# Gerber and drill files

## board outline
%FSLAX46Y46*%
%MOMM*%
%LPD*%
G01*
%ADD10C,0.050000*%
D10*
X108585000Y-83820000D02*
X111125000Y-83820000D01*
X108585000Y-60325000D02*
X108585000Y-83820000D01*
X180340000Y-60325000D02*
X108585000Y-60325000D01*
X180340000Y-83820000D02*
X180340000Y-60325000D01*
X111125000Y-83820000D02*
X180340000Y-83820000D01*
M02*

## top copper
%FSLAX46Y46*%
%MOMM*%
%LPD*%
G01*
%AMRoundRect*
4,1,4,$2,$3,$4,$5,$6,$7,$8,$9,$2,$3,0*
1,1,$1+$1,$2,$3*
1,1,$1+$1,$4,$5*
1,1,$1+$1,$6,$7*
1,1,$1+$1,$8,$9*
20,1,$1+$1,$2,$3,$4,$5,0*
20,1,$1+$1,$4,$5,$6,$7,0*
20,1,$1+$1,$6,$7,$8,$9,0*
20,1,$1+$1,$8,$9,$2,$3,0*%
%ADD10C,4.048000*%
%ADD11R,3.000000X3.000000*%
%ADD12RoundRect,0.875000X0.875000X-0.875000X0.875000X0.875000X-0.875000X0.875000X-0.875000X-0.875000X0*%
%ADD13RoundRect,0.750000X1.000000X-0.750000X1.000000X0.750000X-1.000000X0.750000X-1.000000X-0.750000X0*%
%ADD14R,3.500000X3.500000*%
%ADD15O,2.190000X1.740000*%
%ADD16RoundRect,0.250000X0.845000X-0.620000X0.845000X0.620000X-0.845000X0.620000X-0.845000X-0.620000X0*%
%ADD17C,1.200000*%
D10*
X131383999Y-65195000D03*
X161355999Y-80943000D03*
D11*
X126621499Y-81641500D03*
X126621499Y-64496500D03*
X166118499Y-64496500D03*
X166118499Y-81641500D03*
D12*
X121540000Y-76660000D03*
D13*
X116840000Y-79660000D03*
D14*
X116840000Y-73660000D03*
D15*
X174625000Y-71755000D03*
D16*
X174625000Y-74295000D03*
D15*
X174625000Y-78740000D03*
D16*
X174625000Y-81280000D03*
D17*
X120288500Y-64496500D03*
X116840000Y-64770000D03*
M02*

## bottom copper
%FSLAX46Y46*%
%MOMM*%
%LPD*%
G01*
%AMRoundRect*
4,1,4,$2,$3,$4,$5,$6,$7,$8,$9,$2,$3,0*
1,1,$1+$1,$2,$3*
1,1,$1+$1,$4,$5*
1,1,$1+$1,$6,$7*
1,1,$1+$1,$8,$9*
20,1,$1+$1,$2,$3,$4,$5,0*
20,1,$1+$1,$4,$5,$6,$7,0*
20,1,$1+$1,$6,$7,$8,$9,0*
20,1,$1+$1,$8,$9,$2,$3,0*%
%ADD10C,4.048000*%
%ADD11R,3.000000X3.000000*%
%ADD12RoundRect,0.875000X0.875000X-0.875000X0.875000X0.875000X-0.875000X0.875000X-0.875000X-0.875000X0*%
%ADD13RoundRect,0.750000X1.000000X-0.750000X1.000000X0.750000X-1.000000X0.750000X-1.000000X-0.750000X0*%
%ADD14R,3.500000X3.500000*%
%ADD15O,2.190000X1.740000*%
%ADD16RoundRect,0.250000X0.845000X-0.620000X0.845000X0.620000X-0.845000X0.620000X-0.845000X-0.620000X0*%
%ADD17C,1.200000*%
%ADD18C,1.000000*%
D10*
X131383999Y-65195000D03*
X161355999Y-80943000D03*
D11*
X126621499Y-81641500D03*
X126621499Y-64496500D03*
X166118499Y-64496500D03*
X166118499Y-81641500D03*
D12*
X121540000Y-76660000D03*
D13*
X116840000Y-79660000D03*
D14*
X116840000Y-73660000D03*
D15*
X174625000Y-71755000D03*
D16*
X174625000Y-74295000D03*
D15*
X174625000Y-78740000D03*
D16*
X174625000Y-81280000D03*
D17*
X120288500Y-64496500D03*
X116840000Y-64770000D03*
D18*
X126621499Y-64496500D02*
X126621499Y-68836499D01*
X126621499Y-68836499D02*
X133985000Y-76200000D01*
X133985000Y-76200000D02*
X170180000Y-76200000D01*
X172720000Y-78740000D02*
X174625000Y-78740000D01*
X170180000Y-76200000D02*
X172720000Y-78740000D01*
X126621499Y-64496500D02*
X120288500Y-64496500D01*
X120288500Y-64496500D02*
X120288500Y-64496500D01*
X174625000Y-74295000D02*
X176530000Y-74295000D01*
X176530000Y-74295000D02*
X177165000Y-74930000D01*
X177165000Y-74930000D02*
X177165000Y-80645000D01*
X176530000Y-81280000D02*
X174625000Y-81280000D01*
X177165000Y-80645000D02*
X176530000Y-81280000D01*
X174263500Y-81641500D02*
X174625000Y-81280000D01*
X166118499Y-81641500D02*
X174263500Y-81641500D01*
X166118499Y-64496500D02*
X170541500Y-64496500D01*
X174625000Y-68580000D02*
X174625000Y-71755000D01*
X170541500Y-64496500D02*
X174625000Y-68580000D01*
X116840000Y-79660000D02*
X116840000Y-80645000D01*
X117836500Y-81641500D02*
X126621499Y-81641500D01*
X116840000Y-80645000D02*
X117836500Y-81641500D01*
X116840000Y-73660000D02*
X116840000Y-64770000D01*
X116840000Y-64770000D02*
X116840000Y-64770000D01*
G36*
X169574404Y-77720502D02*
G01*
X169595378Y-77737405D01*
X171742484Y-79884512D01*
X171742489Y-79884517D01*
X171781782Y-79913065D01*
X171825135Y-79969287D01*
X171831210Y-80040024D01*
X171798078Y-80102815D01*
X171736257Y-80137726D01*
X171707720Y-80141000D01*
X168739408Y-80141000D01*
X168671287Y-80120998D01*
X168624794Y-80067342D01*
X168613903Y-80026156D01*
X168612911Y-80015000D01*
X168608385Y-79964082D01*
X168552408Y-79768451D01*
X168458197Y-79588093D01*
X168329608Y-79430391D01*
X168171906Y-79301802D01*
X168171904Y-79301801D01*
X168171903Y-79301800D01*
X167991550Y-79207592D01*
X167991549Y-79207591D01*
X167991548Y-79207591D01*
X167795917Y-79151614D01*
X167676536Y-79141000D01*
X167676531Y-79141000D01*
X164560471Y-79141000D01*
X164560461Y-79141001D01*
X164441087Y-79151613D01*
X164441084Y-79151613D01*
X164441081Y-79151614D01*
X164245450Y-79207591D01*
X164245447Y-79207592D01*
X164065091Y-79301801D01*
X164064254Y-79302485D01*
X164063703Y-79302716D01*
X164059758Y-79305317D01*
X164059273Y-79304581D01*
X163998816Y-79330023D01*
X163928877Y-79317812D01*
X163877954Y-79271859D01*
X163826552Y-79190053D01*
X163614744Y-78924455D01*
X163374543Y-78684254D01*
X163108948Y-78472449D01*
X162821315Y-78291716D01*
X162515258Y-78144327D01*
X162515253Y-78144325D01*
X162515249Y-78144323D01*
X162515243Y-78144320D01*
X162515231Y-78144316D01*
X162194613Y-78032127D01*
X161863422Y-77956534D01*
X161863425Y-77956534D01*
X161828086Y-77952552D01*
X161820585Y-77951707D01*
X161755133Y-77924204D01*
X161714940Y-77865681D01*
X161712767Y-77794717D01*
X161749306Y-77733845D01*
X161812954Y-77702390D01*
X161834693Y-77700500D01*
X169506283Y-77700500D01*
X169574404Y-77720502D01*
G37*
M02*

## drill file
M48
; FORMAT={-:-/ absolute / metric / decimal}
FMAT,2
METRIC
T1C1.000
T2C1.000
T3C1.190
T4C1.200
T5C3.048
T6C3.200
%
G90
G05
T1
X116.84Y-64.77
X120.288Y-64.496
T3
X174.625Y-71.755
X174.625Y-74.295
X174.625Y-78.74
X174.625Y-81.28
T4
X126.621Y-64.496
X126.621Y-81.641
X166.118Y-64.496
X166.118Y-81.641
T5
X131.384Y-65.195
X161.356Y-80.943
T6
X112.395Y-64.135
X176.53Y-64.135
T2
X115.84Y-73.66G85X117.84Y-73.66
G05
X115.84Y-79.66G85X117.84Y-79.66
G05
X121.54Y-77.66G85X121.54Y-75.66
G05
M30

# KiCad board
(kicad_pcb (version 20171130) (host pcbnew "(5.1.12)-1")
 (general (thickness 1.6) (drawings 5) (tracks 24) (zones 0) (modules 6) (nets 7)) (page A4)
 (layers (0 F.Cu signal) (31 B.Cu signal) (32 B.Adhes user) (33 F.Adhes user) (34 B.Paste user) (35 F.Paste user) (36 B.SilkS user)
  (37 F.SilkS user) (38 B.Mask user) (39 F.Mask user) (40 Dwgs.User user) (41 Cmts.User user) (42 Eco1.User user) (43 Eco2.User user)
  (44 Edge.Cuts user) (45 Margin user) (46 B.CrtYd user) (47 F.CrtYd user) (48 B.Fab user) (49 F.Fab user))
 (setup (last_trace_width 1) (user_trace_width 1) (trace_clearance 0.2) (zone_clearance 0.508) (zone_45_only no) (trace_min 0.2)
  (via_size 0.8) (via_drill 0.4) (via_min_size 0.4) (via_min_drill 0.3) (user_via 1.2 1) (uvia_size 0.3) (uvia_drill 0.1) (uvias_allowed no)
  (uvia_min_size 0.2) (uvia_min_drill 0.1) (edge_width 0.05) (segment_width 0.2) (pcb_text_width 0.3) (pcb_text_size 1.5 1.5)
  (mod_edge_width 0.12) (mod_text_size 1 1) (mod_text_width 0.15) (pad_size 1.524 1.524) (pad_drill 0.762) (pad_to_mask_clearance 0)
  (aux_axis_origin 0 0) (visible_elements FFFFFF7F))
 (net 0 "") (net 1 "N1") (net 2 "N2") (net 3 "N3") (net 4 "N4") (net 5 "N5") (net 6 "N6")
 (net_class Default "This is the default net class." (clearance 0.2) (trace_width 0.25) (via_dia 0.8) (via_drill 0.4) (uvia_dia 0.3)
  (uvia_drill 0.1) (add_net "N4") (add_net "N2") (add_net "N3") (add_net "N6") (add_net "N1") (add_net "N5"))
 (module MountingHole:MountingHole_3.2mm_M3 (layer F.Cu) (at 176.53 64.135)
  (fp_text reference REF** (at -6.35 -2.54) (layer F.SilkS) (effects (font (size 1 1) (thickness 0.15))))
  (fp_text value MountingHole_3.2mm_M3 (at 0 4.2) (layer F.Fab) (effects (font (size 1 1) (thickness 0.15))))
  (pad 1 np_thru_hole circle (at 0 0) (size 3.2 3.2) (drill 3.2) (layers *.Cu *.Mask)))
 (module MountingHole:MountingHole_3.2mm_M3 (layer F.Cu) (at 112.395 64.135)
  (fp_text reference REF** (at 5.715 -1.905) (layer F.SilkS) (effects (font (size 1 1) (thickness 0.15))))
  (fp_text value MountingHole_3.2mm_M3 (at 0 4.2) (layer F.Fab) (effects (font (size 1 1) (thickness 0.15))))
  (pad 1 np_thru_hole circle (at 0 0) (size 3.2 3.2) (drill 3.2) (layers *.Cu *.Mask)))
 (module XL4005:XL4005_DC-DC (layer F.Cu) (at 124.779999 83.483)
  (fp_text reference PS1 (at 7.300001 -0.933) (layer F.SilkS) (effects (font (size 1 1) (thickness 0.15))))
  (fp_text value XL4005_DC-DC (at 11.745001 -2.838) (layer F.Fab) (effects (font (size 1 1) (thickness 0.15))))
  (pad "" thru_hole circle (at 6.604 -18.288) (size 4.048 4.048) (drill 3.048) (layers *.Cu *.Mask))
  (pad "" thru_hole circle (at 36.576 -2.54) (size 4.048 4.048) (drill 3.048) (layers *.Cu *.Mask))
  (pad 2 thru_hole rect (at 1.8415 -1.8415) (size 3 3) (drill 1.2) (layers *.Cu *.Mask) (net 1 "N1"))
  (pad 1 thru_hole rect (at 1.8415 -18.9865) (size 3 3) (drill 1.2) (layers *.Cu *.Mask) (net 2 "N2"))
  (pad 3 thru_hole rect (at 41.3385 -18.9865) (size 3 3) (drill 1.2) (layers *.Cu *.Mask) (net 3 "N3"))
  (pad 4 thru_hole rect (at 41.3385 -1.8415) (size 3 3) (drill 1.2) (layers *.Cu *.Mask) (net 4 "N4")))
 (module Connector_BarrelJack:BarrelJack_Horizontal (layer F.Cu) (at 116.84 73.66 90)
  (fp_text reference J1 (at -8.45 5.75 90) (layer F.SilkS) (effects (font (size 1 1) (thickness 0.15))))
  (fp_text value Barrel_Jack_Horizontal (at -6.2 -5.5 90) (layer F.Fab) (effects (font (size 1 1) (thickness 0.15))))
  (pad 3 thru_hole roundrect (at -3 4.7 90) (size 3.5 3.5) (drill oval 3 1) (layers *.Cu *.Mask) (roundrect_rratio 0.25) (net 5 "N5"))
  (pad 2 thru_hole roundrect (at -6 0 90) (size 3 3.5) (drill oval 1 3) (layers *.Cu *.Mask) (roundrect_rratio 0.25) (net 1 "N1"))
  (pad 1 thru_hole rect (at 0 0 90) (size 3.5 3.5) (drill oval 1 3) (layers *.Cu *.Mask) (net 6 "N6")))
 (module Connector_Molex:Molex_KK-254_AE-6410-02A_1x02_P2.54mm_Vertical (layer F.Cu) (at 174.625 74.295 90)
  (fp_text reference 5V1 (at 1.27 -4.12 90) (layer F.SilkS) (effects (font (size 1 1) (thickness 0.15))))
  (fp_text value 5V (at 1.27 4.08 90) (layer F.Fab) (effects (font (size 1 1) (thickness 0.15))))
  (pad 2 thru_hole oval (at 2.54 0 90) (size 1.74 2.19) (drill 1.19) (layers *.Cu *.Mask) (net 3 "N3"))
  (pad 1 thru_hole roundrect (at 0 0 90) (size 1.74 2.19) (drill 1.19) (layers *.Cu *.Mask) (roundrect_rratio 0.143678) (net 4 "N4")))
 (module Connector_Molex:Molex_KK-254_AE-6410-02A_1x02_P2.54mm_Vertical (layer F.Cu) (at 174.625 81.28 90)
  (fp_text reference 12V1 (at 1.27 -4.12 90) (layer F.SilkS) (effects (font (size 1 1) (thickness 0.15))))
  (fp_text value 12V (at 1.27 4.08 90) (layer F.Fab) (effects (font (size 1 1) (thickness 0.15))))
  (pad 2 thru_hole oval (at 2.54 0 90) (size 1.74 2.19) (drill 1.19) (layers *.Cu *.Mask) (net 2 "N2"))
  (pad 1 thru_hole roundrect (at 0 0 90) (size 1.74 2.19) (drill 1.19) (layers *.Cu *.Mask) (roundrect_rratio 0.143678) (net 4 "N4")))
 (gr_line (start 108.585 83.82) (end 111.125 83.82) (layer Edge.Cuts) (width 0.05))
 (gr_line (start 108.585 60.325) (end 108.585 83.82) (layer Edge.Cuts) (width 0.05))
 (gr_line (start 180.34 60.325) (end 108.585 60.325) (layer Edge.Cuts) (width 0.05))
 (gr_line (start 180.34 83.82) (end 180.34 60.325) (layer Edge.Cuts) (width 0.05))
 (gr_line (start 111.125 83.82) (end 180.34 83.82) (layer Edge.Cuts) (width 0.05))
 (segment (start 126.621499 64.4965) (end 126.621499 68.836499) (width 1) (layer B.Cu) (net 2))
 (segment (start 126.621499 68.836499) (end 133.985 76.2) (width 1) (layer B.Cu) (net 2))
 (segment (start 133.985 76.2) (end 170.18 76.2) (width 1) (layer B.Cu) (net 2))
 (segment (start 172.72 78.74) (end 174.625 78.74) (width 1) (layer B.Cu) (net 2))
 (segment (start 170.18 76.2) (end 172.72 78.74) (width 1) (layer B.Cu) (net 2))
 (segment (start 126.621499 64.4965) (end 120.2885 64.4965) (width 1) (layer B.Cu) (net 2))
 (segment (start 120.2885 64.4965) (end 120.2885 64.4965) (width 1) (layer B.Cu) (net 2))
 (via (at 120.2885 64.4965) (size 1.2) (drill 1) (layers F.Cu B.Cu) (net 2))
 (segment (start 174.625 74.295) (end 176.53 74.295) (width 1) (layer B.Cu) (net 4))
 (segment (start 176.53 74.295) (end 177.165 74.93) (width 1) (layer B.Cu) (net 4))
 (segment (start 177.165 74.93) (end 177.165 80.645) (width 1) (layer B.Cu) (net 4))
 (segment (start 176.53 81.28) (end 174.625 81.28) (width 1) (layer B.Cu) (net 4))
 (segment (start 177.165 80.645) (end 176.53 81.28) (width 1) (layer B.Cu) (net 4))
 (segment (start 174.2635 81.6415) (end 174.625 81.28) (width 1) (layer B.Cu) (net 4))
 (segment (start 166.118499 81.6415) (end 174.2635 81.6415) (width 1) (layer B.Cu) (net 4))
 (segment (start 166.118499 64.4965) (end 170.5415 64.4965) (width 1) (layer B.Cu) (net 3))
 (segment (start 174.625 68.58) (end 174.625 71.755) (width 1) (layer B.Cu) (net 3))
 (segment (start 170.5415 64.4965) (end 174.625 68.58) (width 1) (layer B.Cu) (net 3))
 (segment (start 116.84 79.66) (end 116.84 80.645) (width 1) (layer B.Cu) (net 1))
 (segment (start 117.8365 81.6415) (end 126.621499 81.6415) (width 1) (layer B.Cu) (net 1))
 (segment (start 116.84 80.645) (end 117.8365 81.6415) (width 1) (layer B.Cu) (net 1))
 (segment (start 116.84 73.66) (end 116.84 64.77) (width 1) (layer B.Cu) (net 6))
 (segment (start 116.84 64.77) (end 116.84 64.77) (width 1) (layer B.Cu) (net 6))
 (via (at 116.84 64.77) (size 1.2) (drill 1) (layers F.Cu B.Cu) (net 6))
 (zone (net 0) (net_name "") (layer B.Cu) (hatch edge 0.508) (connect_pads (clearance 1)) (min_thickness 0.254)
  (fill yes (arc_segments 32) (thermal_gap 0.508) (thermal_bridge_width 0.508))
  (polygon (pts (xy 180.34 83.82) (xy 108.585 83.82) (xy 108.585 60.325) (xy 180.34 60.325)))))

